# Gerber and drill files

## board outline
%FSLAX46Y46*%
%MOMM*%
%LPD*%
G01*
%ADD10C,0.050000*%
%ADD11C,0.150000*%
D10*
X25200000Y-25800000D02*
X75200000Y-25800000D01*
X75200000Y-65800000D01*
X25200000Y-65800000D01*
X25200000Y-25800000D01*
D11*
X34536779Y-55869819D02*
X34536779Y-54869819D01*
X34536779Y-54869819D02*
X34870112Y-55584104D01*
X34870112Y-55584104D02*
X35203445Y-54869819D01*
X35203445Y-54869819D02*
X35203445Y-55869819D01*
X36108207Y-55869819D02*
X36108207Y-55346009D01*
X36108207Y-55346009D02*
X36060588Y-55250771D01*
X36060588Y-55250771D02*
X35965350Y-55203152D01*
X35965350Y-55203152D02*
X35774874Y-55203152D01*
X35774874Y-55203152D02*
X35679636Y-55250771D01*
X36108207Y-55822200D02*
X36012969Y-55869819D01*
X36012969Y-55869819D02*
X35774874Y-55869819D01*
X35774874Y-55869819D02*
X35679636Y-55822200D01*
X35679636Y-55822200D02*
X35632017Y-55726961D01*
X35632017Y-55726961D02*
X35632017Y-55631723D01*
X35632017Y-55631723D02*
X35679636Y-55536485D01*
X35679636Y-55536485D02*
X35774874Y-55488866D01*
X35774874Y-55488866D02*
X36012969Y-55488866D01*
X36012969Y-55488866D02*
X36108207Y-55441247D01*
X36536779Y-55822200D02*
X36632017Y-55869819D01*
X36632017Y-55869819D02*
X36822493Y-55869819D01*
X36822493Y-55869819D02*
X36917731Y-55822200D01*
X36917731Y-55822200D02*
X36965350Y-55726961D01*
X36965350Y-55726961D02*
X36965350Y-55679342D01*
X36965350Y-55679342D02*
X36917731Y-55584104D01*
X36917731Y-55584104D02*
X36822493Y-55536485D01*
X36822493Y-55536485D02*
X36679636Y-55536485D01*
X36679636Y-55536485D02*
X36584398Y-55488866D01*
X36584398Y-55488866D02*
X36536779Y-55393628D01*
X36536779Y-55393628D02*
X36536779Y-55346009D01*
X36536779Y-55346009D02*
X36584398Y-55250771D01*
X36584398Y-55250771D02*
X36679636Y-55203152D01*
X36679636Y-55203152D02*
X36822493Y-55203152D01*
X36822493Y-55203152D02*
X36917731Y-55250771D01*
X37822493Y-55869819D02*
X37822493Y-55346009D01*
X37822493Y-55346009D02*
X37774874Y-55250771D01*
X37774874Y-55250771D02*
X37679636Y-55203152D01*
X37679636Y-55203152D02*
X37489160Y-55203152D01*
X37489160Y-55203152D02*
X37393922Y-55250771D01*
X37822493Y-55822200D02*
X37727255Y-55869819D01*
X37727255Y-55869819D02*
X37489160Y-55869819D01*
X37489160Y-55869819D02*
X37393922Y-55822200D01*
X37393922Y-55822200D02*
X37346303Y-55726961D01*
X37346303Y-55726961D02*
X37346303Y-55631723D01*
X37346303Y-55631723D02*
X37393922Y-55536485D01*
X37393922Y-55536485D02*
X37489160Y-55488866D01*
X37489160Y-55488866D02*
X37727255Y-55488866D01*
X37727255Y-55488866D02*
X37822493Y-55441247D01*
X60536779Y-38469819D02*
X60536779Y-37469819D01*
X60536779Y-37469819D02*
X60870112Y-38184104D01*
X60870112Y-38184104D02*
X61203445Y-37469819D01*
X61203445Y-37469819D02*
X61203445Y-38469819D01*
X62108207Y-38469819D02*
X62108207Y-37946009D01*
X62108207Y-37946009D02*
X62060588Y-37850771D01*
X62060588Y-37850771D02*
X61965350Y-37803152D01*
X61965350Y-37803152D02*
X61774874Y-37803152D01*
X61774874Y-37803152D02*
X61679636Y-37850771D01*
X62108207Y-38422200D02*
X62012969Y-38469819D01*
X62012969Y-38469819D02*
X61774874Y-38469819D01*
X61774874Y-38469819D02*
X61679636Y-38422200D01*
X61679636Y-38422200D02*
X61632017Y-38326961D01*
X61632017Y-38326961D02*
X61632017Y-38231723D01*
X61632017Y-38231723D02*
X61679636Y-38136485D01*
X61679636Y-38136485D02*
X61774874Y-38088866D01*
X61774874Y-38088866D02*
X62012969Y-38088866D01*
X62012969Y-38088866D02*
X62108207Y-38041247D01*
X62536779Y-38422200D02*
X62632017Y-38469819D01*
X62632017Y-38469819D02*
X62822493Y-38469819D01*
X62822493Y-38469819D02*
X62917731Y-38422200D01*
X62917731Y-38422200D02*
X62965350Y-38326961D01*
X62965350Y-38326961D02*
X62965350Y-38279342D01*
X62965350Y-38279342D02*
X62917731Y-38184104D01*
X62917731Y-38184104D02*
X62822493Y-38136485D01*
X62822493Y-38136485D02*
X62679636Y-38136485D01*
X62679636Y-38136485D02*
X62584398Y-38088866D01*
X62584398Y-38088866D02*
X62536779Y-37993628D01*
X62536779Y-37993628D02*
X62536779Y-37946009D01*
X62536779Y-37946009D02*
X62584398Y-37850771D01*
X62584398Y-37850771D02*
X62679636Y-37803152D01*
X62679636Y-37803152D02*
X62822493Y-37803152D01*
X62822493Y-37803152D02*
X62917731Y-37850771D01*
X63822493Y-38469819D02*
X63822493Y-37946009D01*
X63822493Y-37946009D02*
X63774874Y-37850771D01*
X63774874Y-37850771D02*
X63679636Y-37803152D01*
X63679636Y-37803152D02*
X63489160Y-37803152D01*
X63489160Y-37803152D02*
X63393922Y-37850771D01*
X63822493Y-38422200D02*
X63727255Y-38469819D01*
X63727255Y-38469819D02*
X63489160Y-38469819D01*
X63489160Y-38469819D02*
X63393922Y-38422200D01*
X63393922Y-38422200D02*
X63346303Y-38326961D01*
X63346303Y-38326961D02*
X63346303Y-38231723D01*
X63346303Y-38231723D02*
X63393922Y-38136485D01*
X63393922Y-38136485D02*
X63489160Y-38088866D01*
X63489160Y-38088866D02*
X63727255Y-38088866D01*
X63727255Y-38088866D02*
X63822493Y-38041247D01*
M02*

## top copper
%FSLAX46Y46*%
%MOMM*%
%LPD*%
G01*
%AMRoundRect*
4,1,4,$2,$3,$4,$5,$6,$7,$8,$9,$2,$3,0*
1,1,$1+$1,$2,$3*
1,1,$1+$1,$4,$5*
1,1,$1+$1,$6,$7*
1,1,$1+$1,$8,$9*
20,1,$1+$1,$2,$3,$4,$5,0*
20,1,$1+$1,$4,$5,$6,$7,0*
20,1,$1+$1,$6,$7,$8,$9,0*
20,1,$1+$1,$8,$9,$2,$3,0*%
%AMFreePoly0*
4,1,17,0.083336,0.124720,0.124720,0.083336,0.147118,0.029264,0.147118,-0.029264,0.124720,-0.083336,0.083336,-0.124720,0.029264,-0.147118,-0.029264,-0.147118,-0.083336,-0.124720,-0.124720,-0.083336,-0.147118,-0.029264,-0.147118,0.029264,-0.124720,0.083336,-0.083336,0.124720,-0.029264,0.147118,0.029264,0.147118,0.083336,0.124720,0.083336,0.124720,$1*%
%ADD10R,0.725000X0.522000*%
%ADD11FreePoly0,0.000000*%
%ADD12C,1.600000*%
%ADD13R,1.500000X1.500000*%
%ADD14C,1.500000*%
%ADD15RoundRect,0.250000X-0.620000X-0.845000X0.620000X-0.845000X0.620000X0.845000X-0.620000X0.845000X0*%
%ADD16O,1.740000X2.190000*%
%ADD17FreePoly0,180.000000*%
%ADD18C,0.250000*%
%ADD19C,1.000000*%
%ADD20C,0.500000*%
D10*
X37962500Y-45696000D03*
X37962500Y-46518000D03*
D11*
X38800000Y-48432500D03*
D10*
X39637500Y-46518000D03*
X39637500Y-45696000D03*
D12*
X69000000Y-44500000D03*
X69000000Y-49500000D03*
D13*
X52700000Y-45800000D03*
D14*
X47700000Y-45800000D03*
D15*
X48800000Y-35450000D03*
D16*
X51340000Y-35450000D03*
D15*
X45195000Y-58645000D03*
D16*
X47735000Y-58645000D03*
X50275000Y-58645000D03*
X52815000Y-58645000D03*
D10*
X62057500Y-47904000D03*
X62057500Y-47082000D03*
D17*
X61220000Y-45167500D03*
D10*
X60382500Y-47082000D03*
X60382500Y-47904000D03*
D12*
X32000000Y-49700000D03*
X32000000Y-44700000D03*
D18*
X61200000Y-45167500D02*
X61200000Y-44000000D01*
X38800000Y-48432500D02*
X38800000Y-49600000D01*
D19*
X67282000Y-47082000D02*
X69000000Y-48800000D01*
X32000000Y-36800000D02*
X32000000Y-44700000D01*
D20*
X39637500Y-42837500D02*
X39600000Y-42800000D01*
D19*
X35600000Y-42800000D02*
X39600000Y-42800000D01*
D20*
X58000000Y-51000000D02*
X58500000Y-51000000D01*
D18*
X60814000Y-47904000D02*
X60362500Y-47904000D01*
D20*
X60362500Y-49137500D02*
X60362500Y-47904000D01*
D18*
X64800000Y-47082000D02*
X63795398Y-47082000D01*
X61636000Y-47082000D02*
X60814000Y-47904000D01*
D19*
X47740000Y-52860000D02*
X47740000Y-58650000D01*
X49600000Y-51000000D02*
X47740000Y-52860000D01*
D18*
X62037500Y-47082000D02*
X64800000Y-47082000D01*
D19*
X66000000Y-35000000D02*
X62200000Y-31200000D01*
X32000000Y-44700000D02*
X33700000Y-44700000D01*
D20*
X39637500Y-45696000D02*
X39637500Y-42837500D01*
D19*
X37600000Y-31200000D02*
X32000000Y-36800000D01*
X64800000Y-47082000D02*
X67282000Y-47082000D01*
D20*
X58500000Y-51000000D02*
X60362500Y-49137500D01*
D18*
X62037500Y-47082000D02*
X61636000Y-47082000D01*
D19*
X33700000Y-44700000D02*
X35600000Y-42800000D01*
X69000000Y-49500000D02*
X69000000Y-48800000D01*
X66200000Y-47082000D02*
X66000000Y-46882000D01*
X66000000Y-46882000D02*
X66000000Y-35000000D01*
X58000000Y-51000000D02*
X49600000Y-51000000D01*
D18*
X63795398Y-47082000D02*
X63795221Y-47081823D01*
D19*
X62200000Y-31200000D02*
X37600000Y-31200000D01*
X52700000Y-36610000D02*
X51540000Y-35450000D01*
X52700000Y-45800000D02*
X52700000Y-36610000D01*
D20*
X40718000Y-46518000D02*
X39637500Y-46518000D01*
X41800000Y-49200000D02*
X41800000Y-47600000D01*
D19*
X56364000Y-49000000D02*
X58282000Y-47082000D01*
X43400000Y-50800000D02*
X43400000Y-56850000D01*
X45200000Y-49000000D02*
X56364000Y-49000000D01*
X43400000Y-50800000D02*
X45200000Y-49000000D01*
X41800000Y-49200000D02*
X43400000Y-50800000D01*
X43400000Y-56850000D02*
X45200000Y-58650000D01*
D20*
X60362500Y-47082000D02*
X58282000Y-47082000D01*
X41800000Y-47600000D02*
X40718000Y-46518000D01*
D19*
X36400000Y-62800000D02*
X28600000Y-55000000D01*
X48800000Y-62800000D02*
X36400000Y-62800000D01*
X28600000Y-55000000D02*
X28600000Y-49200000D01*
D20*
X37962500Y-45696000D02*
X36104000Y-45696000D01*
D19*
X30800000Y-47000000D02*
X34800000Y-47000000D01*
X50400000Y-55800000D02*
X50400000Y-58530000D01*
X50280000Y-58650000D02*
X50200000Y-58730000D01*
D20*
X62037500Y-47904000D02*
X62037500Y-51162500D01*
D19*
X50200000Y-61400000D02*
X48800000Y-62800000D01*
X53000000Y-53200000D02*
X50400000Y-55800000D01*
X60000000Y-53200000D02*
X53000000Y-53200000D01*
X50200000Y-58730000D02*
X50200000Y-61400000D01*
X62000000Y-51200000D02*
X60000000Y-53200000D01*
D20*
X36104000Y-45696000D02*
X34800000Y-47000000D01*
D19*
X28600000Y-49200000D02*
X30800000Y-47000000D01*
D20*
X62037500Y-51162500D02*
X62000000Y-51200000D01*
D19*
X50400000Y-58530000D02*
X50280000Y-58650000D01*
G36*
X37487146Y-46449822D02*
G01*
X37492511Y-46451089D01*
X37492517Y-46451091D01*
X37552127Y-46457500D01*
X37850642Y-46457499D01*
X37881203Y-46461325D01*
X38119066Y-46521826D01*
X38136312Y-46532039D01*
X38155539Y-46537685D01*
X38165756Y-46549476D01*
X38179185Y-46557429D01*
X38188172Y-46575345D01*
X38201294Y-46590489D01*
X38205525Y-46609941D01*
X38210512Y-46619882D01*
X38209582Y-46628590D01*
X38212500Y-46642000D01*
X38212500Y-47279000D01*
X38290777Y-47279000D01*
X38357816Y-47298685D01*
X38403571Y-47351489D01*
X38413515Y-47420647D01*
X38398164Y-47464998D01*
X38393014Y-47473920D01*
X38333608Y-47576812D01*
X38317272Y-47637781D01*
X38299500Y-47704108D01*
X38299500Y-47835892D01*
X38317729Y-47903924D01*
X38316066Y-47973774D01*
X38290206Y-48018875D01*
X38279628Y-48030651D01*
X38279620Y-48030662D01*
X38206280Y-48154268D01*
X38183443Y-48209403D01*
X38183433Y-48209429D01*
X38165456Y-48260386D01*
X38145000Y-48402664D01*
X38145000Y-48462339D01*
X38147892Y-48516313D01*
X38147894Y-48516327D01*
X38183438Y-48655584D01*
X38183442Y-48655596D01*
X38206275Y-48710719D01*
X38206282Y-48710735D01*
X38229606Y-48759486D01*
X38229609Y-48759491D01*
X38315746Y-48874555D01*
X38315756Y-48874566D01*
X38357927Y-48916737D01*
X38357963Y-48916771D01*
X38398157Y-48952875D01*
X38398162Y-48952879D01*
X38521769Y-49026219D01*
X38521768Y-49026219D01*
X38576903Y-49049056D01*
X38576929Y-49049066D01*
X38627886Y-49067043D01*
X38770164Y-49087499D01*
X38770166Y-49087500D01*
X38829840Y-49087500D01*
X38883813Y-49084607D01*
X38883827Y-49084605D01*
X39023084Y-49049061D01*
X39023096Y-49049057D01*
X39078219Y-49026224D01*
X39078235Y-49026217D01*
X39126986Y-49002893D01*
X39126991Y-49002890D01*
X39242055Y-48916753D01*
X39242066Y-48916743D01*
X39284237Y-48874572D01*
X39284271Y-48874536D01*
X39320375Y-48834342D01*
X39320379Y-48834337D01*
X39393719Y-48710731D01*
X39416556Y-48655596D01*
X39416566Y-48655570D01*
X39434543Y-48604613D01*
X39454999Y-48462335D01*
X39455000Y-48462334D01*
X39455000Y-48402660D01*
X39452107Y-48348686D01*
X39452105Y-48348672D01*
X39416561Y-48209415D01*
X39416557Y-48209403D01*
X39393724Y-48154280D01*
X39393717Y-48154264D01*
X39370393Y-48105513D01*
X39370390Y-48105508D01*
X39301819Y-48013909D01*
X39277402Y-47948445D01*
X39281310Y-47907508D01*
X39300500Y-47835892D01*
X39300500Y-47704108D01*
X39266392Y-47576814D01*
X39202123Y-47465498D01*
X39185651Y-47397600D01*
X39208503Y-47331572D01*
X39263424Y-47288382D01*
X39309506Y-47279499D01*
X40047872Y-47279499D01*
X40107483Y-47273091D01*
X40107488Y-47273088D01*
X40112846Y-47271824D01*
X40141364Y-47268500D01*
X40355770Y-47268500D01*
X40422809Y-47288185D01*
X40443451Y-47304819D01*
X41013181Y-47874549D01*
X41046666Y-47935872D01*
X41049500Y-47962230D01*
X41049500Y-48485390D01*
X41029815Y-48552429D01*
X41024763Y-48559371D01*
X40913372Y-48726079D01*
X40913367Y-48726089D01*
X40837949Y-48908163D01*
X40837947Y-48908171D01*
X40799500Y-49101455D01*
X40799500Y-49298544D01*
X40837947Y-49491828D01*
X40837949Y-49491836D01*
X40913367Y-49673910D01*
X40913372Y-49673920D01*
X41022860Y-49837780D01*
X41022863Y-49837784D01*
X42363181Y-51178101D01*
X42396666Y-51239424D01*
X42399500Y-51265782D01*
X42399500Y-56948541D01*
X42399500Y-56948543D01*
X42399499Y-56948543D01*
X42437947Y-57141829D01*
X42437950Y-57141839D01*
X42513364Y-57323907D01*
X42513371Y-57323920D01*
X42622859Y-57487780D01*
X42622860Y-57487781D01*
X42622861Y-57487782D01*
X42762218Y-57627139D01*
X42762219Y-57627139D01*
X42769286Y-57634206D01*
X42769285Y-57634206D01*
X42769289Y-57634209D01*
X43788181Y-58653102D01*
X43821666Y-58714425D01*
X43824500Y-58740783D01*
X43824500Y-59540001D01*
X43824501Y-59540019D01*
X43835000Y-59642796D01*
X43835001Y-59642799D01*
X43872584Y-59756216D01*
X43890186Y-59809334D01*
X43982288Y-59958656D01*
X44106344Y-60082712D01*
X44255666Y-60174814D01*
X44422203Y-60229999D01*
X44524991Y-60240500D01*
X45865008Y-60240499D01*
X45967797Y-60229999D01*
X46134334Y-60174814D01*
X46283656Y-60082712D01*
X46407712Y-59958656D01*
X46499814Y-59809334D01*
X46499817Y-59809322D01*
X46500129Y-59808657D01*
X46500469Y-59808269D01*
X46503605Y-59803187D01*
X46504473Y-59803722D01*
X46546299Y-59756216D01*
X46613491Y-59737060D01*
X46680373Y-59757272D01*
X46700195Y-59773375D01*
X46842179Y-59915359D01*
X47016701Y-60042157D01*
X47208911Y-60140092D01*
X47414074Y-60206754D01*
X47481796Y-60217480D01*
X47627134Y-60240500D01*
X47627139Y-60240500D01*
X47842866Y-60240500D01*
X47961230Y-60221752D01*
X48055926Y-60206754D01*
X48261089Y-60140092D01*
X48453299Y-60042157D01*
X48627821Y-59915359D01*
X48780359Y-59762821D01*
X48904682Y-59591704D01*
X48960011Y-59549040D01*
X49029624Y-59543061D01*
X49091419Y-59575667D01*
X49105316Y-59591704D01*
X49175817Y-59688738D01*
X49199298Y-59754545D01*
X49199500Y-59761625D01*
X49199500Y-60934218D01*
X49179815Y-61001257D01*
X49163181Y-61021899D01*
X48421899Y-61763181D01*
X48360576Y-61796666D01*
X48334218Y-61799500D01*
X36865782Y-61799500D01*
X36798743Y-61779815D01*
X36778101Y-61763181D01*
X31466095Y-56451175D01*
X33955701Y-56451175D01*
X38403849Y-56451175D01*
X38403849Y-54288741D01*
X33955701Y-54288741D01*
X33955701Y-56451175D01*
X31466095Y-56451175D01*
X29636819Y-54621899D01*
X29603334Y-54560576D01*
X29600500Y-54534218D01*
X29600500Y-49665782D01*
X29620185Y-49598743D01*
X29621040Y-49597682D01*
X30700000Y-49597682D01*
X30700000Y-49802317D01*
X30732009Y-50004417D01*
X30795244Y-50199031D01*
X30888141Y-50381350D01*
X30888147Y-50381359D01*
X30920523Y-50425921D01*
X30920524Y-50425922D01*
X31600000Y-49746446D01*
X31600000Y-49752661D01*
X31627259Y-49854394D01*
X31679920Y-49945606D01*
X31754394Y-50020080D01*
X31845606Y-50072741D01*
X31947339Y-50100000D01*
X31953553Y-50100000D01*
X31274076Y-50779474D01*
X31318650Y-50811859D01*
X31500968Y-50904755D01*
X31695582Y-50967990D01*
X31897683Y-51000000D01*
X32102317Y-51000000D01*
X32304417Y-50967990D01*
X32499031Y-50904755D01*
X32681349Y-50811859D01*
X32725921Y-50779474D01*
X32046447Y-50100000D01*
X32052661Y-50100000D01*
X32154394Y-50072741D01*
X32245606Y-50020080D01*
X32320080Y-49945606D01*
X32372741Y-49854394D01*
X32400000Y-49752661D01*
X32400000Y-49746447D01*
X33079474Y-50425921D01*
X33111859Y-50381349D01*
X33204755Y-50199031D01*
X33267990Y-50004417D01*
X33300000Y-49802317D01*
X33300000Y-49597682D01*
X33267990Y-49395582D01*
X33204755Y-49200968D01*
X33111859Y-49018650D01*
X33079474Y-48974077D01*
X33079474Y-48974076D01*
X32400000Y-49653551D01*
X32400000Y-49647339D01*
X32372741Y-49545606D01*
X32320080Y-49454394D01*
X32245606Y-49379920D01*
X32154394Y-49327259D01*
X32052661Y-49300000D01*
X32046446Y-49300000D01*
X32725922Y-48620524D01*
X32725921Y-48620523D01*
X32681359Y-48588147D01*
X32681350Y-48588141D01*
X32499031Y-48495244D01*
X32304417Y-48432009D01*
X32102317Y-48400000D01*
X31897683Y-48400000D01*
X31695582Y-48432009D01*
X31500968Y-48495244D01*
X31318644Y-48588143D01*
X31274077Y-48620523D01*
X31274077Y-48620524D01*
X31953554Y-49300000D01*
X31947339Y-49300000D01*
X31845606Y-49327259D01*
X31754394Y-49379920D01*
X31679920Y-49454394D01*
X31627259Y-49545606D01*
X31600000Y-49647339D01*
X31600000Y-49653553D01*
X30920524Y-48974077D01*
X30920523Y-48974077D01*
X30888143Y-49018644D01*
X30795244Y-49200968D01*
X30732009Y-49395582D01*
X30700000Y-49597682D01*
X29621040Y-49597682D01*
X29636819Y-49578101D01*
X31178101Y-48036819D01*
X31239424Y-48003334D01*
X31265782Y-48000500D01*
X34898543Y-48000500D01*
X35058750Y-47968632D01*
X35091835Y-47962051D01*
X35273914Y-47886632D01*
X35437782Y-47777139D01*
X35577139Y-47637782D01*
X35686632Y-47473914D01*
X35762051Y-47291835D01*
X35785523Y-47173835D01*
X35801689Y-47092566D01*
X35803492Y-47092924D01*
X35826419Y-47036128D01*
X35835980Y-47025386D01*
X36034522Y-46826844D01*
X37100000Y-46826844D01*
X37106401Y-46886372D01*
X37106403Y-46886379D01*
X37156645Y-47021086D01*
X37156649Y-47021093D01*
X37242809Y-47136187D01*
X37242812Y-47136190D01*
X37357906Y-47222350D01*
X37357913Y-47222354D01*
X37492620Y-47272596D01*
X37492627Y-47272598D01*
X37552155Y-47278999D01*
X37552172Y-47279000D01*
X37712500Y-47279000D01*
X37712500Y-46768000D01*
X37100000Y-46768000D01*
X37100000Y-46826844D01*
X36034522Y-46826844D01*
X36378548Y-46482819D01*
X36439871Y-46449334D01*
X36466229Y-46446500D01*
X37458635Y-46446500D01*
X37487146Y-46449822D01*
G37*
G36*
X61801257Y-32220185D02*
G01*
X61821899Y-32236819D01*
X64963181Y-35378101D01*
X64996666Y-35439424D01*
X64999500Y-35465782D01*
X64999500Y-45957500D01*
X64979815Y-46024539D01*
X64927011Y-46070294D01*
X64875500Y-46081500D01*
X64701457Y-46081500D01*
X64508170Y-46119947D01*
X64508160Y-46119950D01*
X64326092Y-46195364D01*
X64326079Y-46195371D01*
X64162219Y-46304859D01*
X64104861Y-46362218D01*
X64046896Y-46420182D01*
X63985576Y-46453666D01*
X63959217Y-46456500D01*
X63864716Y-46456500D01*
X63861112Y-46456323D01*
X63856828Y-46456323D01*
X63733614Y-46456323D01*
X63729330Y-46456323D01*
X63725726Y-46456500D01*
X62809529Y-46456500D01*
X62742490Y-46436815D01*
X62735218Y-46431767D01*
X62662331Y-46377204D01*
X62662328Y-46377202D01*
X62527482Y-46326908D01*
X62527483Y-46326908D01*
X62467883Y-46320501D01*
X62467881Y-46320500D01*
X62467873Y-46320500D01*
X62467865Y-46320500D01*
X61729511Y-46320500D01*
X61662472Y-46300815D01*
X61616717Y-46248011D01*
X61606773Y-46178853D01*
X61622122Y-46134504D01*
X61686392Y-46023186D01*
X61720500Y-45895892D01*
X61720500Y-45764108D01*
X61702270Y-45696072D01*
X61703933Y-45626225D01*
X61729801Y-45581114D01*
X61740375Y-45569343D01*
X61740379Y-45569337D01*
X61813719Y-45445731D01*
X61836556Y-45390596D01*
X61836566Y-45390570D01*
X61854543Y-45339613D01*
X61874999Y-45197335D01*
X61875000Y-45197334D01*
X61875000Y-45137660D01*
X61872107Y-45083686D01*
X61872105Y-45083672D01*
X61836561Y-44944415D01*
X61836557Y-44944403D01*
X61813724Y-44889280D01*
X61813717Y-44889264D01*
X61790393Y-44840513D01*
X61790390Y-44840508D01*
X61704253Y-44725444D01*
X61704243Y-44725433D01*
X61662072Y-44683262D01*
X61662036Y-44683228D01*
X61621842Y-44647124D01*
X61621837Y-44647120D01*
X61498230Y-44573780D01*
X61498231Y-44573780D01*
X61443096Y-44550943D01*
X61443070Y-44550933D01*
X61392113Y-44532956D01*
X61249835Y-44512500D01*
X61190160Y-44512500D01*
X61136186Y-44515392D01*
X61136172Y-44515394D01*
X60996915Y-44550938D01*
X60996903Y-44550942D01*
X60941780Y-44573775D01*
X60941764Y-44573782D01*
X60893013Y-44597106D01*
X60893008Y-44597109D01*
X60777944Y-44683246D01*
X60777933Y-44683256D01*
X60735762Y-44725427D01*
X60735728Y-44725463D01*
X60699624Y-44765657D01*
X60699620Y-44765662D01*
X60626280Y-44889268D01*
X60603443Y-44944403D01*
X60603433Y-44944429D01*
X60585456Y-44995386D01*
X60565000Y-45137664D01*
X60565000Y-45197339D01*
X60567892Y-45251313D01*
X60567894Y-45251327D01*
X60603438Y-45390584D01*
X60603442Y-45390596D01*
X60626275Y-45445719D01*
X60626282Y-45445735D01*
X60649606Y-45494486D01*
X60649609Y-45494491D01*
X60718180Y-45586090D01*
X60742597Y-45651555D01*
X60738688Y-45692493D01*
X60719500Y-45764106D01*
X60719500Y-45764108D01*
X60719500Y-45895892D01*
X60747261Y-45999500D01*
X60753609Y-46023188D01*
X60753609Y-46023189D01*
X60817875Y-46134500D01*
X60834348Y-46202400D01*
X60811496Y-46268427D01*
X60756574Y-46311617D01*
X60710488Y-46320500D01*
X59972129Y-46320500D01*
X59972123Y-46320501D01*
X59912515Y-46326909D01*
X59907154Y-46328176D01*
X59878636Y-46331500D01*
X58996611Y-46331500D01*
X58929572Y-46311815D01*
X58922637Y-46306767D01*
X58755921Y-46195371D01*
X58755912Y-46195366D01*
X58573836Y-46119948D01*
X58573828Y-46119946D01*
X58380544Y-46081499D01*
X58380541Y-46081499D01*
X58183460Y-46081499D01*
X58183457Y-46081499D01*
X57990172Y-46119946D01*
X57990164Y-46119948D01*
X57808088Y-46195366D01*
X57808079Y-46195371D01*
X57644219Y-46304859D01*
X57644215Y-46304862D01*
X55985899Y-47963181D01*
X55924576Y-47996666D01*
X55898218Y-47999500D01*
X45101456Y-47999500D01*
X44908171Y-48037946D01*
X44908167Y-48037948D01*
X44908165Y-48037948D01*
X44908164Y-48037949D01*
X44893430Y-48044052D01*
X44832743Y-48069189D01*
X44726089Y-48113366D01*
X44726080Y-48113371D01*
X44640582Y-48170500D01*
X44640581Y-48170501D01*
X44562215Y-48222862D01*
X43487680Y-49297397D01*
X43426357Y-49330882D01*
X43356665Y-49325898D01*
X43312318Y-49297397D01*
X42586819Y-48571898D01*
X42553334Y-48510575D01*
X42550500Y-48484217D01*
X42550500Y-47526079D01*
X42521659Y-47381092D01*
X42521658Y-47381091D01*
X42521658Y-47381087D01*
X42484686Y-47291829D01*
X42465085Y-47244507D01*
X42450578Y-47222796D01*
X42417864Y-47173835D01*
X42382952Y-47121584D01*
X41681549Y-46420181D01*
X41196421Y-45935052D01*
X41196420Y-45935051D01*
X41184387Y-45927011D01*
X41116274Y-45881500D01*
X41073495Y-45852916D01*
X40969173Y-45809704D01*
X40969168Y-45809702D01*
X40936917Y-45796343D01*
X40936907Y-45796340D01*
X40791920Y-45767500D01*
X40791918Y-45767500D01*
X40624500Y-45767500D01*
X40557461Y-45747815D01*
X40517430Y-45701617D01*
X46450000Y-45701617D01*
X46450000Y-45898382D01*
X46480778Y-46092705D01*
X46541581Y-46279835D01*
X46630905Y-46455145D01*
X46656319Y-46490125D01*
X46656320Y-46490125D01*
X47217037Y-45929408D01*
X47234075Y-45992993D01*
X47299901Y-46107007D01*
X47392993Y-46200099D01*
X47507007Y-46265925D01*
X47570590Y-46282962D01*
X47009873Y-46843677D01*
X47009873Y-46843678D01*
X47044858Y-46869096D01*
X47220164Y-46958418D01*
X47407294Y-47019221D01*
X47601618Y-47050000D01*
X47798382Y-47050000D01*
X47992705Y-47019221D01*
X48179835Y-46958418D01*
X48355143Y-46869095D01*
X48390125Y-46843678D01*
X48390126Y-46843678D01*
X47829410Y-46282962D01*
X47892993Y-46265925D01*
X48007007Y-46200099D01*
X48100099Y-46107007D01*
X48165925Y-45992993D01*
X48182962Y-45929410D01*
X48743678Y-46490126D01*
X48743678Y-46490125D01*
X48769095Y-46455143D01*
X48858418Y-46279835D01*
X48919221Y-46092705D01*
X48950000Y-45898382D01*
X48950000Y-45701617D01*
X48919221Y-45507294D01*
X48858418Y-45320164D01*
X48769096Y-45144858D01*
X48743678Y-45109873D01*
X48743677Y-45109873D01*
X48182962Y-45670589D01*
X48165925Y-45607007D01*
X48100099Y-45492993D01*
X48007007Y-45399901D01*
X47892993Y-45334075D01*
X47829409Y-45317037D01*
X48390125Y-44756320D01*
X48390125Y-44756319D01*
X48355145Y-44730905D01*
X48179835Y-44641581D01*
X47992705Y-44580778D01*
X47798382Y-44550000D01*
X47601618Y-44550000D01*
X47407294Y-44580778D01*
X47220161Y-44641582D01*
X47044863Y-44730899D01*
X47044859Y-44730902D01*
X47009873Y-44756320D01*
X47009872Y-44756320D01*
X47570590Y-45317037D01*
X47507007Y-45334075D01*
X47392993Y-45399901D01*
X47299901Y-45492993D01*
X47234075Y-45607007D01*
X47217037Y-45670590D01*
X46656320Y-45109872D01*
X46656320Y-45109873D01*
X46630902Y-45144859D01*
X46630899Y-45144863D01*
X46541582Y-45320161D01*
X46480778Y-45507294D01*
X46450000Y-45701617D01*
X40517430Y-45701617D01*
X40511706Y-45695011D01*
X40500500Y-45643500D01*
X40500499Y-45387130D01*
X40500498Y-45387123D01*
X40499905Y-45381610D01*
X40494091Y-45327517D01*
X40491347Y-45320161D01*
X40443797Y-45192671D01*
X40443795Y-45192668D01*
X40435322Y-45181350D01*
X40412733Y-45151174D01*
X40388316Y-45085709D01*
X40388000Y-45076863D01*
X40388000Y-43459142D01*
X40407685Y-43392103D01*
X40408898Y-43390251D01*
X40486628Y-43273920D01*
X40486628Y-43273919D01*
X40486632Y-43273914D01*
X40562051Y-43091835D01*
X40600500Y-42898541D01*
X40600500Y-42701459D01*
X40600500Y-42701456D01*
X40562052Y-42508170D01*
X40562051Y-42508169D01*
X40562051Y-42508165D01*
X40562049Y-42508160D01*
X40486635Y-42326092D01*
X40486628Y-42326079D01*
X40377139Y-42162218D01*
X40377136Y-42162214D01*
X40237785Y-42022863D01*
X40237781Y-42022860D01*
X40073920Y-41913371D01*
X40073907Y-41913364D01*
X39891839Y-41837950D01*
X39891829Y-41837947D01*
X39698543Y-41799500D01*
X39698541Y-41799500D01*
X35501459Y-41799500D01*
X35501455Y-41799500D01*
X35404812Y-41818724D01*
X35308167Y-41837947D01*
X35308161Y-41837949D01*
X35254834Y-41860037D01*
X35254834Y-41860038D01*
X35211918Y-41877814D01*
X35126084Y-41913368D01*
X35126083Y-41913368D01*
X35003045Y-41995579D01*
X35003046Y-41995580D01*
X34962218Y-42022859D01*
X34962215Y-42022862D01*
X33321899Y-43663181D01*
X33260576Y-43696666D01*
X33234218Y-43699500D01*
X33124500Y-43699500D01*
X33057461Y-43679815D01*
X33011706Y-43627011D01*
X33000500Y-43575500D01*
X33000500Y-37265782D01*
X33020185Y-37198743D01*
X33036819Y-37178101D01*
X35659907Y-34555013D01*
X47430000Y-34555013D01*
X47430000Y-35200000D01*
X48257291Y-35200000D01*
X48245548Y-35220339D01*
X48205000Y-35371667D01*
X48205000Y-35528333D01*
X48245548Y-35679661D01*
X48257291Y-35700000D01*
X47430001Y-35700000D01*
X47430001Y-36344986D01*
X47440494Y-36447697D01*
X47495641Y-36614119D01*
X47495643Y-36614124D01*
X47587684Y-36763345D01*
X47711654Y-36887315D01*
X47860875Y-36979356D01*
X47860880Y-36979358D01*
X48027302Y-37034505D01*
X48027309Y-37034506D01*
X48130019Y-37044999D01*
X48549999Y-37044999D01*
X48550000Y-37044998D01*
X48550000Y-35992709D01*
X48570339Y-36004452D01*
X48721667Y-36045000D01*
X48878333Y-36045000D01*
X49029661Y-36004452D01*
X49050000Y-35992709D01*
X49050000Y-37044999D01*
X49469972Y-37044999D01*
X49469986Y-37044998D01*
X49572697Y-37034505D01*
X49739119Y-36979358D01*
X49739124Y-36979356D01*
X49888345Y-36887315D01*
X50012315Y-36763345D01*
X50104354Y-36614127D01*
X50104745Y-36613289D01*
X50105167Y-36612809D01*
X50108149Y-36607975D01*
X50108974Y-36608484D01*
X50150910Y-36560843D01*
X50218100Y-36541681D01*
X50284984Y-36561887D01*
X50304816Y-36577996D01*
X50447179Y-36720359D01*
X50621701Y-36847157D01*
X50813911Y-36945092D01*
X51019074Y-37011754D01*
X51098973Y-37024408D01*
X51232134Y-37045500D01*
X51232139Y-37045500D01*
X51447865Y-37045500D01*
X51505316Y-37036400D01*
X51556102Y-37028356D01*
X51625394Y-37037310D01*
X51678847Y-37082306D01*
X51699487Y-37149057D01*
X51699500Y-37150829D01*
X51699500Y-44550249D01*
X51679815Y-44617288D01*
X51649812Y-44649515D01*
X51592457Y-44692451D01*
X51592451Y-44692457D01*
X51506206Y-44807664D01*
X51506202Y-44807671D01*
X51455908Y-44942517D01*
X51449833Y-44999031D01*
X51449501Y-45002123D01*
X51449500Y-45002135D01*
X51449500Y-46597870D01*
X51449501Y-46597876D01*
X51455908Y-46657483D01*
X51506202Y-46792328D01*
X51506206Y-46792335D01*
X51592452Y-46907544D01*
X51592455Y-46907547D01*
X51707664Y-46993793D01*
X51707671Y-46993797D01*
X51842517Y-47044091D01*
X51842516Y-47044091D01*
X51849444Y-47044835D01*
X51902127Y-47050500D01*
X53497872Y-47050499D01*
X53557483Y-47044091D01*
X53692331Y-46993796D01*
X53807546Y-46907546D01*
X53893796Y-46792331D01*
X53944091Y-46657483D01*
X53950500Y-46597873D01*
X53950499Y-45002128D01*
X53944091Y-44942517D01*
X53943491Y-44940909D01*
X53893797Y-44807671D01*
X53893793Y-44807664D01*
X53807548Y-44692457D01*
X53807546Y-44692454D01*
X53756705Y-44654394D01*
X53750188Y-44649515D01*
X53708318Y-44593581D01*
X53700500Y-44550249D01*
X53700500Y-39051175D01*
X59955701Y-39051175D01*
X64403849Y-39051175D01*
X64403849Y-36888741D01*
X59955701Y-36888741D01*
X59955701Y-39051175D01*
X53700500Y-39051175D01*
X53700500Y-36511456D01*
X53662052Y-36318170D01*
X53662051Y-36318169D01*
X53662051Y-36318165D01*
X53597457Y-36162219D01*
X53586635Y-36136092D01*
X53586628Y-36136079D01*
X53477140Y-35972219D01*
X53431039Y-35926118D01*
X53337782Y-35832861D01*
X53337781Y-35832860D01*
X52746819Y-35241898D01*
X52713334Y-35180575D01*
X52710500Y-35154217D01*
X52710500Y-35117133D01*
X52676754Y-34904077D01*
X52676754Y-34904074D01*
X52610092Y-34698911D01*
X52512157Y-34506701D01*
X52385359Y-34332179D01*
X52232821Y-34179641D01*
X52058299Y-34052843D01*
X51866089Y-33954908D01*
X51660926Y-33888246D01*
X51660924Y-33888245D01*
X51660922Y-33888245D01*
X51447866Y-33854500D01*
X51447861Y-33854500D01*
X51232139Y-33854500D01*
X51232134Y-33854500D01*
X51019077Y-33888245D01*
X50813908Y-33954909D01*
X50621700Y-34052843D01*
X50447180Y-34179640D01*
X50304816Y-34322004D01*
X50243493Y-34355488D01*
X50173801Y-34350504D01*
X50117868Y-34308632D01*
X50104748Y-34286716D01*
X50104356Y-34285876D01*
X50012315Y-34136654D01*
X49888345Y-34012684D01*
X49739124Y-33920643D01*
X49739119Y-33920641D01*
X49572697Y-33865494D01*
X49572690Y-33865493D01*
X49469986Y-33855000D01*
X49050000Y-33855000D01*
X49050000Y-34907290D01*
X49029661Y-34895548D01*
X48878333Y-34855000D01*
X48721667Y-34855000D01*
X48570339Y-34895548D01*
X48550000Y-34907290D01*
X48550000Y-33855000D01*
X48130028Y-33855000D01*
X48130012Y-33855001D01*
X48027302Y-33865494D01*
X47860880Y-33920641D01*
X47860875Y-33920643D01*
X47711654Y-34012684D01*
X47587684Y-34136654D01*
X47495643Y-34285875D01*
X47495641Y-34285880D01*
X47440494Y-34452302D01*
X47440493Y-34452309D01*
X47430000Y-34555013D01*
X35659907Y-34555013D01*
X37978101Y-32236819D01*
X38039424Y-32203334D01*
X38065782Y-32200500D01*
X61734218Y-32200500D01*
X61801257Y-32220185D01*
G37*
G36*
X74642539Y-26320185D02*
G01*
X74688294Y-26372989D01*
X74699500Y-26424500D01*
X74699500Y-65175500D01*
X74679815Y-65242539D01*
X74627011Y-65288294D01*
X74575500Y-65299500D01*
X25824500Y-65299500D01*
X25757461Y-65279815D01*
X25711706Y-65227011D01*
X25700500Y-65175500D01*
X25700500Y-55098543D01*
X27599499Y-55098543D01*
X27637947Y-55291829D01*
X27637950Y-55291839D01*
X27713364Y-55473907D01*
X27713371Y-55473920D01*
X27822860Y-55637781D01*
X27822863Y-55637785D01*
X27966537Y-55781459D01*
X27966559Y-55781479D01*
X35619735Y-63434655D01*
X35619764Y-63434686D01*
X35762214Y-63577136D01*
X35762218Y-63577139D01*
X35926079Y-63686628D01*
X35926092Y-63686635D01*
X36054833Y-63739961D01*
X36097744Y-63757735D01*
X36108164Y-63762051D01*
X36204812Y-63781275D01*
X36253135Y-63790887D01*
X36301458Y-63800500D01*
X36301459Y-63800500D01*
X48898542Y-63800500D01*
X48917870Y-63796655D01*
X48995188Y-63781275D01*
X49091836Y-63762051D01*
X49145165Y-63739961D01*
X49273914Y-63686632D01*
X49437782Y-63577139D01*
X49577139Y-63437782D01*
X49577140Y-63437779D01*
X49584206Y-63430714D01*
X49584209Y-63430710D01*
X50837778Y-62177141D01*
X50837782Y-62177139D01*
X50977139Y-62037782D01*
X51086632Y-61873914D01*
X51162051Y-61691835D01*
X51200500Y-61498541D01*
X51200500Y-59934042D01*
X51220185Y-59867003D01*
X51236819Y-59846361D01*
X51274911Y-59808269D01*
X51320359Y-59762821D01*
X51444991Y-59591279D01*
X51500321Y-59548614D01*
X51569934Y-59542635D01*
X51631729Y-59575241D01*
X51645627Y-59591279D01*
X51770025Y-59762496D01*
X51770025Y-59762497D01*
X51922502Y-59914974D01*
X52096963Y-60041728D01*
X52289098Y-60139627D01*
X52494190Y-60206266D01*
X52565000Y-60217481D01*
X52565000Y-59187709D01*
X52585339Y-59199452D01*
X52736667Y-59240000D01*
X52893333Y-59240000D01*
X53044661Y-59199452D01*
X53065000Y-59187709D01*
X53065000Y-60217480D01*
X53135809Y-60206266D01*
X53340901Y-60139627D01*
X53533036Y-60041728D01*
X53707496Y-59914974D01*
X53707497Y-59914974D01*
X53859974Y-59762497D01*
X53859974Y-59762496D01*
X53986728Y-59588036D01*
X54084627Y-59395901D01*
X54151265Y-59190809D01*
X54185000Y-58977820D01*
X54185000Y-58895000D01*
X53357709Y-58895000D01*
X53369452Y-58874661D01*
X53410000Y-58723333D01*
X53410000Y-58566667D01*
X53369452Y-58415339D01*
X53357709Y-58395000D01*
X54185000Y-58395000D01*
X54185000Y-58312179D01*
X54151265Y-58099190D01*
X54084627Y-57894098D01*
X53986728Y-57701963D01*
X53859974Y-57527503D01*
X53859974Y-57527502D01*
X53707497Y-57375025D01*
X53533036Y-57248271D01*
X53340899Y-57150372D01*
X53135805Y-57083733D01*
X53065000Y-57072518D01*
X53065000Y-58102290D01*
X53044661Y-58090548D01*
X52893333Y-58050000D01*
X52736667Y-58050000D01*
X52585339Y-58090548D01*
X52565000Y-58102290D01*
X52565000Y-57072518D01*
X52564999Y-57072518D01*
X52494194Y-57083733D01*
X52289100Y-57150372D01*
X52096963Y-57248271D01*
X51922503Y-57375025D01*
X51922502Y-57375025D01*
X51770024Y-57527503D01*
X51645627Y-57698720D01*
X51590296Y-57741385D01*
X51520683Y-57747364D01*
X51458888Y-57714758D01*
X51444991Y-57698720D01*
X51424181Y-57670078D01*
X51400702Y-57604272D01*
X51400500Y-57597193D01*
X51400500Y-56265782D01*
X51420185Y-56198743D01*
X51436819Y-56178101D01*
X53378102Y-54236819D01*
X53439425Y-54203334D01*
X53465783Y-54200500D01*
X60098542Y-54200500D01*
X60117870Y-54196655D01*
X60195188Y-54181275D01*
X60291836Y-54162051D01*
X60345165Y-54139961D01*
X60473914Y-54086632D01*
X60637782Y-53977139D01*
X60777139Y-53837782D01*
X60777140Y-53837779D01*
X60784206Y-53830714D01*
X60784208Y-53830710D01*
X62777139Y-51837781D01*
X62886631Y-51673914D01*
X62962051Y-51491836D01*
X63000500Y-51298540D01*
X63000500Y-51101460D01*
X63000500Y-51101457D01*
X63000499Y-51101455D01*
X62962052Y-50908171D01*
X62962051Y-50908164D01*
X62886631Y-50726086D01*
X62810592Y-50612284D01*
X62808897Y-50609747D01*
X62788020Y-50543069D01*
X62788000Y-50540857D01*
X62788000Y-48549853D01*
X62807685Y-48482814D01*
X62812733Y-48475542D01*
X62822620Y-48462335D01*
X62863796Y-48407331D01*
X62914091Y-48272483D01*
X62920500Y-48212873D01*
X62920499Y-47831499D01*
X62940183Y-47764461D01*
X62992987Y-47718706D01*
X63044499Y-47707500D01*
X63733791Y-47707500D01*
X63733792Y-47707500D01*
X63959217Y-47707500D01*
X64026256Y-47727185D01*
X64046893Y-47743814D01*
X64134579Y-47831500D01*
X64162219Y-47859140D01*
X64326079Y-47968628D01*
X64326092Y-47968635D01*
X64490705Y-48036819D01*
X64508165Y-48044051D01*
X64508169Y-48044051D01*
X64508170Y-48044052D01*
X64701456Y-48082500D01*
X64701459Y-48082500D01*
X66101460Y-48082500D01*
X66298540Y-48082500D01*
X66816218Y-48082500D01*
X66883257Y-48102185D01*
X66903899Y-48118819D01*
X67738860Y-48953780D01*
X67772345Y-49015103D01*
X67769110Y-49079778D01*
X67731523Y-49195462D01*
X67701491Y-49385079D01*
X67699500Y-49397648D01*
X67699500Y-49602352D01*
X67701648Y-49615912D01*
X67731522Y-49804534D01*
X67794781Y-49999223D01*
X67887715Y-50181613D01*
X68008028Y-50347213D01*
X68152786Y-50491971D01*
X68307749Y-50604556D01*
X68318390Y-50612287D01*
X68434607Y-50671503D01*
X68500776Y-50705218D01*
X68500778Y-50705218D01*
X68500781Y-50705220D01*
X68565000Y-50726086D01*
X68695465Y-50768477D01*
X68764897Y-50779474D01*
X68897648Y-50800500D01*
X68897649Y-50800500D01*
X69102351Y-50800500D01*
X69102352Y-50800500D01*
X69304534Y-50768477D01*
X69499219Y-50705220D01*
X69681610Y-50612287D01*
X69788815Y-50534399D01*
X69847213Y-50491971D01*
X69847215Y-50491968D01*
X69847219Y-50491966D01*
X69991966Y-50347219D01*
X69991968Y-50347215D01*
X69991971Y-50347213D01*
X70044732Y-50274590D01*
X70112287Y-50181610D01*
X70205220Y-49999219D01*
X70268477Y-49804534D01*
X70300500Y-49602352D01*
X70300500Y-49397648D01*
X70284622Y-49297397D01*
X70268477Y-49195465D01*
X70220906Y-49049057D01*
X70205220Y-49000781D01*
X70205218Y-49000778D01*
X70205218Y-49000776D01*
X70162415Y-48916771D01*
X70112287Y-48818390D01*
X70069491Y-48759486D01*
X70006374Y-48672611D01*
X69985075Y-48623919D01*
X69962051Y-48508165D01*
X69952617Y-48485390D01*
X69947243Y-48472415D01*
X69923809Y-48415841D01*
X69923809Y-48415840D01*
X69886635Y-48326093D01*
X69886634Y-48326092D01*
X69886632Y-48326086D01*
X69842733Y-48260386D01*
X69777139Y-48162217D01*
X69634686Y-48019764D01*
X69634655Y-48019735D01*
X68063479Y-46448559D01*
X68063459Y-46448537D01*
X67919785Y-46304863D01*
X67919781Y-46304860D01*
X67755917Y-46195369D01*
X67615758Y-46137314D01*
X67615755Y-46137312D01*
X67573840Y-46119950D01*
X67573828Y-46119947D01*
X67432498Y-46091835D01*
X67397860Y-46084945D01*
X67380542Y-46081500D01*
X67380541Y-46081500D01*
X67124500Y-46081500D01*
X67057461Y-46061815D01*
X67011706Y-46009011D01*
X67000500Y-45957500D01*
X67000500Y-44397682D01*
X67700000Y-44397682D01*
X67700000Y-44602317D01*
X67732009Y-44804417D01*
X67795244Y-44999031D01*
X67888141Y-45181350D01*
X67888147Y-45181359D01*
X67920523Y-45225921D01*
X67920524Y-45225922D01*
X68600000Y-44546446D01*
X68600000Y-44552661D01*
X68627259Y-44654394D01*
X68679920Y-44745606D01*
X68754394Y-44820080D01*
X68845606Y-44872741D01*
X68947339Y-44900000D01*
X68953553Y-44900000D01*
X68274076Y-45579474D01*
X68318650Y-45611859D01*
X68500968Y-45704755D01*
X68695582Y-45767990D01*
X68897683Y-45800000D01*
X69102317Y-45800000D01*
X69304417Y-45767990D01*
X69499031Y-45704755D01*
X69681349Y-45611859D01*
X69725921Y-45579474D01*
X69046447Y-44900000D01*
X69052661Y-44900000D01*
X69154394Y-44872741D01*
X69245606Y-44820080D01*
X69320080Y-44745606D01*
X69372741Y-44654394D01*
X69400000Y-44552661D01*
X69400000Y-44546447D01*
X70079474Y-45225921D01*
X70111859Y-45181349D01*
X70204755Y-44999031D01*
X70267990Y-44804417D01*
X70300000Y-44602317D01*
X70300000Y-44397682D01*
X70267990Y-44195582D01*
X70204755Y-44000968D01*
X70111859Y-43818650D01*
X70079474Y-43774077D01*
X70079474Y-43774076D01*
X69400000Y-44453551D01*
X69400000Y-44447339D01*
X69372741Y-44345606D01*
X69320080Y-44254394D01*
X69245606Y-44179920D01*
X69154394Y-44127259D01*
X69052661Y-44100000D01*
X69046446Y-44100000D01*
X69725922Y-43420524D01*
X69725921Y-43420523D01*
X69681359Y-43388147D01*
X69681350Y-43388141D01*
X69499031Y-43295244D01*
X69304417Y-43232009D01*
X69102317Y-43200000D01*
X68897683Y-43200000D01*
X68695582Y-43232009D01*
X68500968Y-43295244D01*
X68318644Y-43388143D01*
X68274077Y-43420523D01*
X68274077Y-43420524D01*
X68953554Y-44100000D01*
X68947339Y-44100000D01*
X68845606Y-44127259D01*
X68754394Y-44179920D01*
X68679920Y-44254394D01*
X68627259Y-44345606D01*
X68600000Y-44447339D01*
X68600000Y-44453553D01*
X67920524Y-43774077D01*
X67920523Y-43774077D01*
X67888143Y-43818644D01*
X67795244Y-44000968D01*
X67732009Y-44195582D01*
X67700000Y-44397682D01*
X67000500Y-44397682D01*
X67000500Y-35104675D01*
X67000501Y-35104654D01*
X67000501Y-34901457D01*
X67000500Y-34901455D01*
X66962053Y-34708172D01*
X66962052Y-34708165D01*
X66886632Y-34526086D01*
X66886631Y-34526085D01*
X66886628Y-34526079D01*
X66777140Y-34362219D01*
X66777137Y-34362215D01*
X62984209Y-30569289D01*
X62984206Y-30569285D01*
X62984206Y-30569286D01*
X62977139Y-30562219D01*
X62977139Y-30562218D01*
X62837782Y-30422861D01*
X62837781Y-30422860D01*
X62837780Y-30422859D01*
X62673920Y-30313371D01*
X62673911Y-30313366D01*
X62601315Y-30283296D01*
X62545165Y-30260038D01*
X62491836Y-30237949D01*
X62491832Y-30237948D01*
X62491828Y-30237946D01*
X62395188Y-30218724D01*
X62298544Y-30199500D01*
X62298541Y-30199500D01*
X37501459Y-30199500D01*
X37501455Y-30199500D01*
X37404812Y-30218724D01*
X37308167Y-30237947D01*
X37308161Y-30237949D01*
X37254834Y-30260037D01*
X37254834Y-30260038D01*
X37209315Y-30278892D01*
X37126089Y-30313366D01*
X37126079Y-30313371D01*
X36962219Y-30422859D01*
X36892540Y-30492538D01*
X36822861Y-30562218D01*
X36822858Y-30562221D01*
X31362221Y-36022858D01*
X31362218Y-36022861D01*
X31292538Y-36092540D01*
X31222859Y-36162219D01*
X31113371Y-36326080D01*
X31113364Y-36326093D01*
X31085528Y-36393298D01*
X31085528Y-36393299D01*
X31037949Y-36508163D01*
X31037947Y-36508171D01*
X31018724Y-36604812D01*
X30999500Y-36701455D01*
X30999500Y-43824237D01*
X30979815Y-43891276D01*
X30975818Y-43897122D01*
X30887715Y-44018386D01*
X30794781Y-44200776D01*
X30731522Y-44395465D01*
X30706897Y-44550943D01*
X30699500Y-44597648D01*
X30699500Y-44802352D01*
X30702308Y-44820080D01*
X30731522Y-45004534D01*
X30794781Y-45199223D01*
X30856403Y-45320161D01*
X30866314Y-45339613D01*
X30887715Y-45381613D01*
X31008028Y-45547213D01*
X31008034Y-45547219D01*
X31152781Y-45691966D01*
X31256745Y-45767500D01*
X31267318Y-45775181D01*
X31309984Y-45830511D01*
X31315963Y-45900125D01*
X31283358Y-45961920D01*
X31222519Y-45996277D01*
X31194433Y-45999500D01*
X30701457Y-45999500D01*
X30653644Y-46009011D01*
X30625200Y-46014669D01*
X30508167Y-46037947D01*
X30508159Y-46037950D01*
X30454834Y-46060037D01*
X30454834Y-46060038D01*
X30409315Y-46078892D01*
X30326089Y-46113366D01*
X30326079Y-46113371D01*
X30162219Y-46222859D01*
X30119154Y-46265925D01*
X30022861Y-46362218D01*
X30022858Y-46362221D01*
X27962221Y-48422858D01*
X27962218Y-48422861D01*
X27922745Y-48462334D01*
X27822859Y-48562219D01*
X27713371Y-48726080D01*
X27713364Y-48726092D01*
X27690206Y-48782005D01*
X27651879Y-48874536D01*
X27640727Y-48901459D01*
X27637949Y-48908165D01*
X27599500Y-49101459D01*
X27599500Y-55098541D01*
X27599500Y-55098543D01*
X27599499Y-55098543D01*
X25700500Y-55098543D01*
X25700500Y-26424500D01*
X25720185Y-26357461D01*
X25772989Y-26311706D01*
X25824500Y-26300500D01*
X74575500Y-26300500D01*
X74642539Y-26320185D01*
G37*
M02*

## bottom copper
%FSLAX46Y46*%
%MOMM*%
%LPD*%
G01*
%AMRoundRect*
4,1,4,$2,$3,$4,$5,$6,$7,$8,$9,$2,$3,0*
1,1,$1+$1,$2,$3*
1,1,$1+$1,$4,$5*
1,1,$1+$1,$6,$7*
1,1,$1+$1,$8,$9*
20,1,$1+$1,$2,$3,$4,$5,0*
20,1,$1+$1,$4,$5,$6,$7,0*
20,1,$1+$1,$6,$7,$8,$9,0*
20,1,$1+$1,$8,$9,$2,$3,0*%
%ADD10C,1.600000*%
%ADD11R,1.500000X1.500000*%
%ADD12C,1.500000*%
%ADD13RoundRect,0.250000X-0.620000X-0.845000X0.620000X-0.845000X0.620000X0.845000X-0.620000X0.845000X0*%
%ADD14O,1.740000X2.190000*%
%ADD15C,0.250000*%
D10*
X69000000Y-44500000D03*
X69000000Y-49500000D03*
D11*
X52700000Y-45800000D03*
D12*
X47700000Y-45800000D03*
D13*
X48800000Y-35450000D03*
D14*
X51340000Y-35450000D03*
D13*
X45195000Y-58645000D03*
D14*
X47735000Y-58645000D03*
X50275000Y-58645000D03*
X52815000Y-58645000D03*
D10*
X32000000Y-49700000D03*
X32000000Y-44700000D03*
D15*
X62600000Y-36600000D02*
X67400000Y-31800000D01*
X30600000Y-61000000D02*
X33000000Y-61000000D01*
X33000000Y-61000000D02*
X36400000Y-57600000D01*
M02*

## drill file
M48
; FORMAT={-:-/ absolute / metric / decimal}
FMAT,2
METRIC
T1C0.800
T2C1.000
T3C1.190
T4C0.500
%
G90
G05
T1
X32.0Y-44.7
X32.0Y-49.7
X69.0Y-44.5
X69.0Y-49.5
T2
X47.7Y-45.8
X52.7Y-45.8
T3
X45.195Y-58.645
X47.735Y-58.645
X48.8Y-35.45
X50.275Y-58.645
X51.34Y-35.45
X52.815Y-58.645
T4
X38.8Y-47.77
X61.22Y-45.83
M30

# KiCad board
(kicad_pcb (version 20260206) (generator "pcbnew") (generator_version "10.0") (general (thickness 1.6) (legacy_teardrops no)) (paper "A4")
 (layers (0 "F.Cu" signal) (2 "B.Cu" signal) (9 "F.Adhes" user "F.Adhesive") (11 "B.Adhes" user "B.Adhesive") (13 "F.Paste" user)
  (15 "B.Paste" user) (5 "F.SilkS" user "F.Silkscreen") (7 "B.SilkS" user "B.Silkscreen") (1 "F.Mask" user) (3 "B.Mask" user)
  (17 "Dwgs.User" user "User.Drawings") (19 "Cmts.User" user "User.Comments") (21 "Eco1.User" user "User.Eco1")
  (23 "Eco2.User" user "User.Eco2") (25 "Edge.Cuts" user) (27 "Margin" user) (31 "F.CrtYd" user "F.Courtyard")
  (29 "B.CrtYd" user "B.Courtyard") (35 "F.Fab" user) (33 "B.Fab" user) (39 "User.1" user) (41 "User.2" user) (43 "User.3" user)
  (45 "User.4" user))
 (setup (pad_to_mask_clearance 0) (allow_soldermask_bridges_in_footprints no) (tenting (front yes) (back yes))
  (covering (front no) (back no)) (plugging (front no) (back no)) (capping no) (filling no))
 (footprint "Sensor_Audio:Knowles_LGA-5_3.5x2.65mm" (layer "F.Cu") (at 38.8 47)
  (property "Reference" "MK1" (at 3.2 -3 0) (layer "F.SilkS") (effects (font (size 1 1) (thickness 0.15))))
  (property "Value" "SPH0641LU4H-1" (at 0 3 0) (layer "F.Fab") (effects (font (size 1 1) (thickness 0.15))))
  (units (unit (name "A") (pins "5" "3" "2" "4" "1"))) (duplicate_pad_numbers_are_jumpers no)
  (pad "" np_thru_hole circle (at 0 0.77) (size 0.5 0.5) (drill 0.5) (layers "*.Cu" "*.Mask"))
  (pad "1" smd rect (at -0.8375 -1.304) (size 0.725 0.522) (layers "F.Cu" "F.Mask" "F.Paste") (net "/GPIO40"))
  (pad "2" smd rect (at -0.8375 -0.482) (size 0.725 0.522) (layers "F.Cu" "F.Mask" "F.Paste") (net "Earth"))
  (pad "3" smd custom (at 0 1.4325) (size 0.3 0.3) (layers "F.Cu" "F.Mask") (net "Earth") (zone_connect 0)
   (options (clearance outline) (anchor circle)) (primitives))
  (pad "4" smd rect (at 0.8375 -0.482) (size 0.725 0.522) (layers "F.Cu" "F.Mask" "F.Paste") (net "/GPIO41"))
  (pad "5" smd rect (at 0.8375 -1.304) (size 0.725 0.522) (layers "F.Cu" "F.Mask" "F.Paste") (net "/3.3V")))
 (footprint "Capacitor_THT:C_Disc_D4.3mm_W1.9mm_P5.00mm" (layer "F.Cu") (at 69 44.5 -90)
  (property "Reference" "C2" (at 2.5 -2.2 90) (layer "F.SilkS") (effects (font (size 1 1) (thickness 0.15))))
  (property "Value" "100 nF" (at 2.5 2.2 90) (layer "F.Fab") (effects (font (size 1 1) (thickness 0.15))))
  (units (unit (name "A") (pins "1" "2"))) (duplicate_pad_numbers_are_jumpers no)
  (pad "1" thru_hole circle (at 0 0 270) (size 1.6 1.6) (drill 0.8) (layers "*.Cu" "*.Mask") (remove_unused_layers no) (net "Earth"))
  (pad "2" thru_hole circle (at 5 0 270) (size 1.6 1.6) (drill 0.8) (layers "*.Cu" "*.Mask") (remove_unused_layers no) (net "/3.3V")))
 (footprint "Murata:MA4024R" (layer "F.Cu") (at 50.2 45.8 180)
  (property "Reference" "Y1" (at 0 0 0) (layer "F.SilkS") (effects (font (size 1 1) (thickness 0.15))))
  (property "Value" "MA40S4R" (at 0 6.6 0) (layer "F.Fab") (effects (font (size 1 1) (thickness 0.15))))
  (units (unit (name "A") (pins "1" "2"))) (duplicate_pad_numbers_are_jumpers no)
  (pad "1" thru_hole rect (at -2.5 0 180) (size 1.5 1.5) (drill 1) (layers "*.Cu" "*.Mask") (remove_unused_layers no)
   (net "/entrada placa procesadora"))
  (pad "2" thru_hole circle (at 2.5 0 180) (size 1.5 1.5) (drill 1) (layers "*.Cu" "*.Mask") (remove_unused_layers no) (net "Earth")))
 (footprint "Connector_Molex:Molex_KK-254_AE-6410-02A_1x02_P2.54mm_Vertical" (layer "F.Cu") (at 48.8 35.45)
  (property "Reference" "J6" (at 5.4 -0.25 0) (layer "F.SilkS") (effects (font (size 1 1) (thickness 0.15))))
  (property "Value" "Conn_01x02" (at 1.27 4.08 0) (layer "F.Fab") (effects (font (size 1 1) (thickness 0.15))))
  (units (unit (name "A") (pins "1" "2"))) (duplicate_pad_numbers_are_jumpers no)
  (pad "1" thru_hole roundrect (at 0 0) (size 1.74 2.19) (drill 1.19) (layers "*.Cu" "*.Mask") (remove_unused_layers no)
   (roundrect_rratio 0.143678) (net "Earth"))
  (pad "2" thru_hole oval (at 2.54 0) (size 1.74 2.19) (drill 1.19) (layers "*.Cu" "*.Mask") (remove_unused_layers no)
   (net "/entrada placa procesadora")))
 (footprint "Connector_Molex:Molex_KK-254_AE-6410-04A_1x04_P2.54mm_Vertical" (layer "F.Cu") (at 45.195 58.645)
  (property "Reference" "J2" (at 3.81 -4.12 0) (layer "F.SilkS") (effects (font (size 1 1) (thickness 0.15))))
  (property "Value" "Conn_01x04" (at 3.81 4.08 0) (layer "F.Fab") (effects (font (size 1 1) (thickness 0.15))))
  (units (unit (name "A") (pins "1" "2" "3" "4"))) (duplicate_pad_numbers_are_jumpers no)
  (pad "1" thru_hole roundrect (at 0 0) (size 1.74 2.19) (drill 1.19) (layers "*.Cu" "*.Mask") (remove_unused_layers no)
   (roundrect_rratio 0.143678) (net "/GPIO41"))
  (pad "2" thru_hole oval (at 2.54 0) (size 1.74 2.19) (drill 1.19) (layers "*.Cu" "*.Mask") (remove_unused_layers no) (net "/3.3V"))
  (pad "3" thru_hole oval (at 5.08 0) (size 1.74 2.19) (drill 1.19) (layers "*.Cu" "*.Mask") (remove_unused_layers no) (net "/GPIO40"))
  (pad "4" thru_hole oval (at 7.62 0) (size 1.74 2.19) (drill 1.19) (layers "*.Cu" "*.Mask") (remove_unused_layers no) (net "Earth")))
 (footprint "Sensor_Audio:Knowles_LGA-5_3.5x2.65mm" (layer "F.Cu") (at 61.22 46.6 180)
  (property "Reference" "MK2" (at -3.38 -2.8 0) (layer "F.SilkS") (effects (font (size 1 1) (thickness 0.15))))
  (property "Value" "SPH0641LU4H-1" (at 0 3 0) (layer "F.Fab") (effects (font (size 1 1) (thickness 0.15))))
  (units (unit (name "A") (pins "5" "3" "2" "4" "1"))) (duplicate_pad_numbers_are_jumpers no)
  (pad "" np_thru_hole circle (at 0 0.77 180) (size 0.5 0.5) (drill 0.5) (layers "*.Cu" "*.Mask"))
  (pad "1" smd rect (at -0.8375 -1.304 180) (size 0.725 0.522) (layers "F.Cu" "F.Mask" "F.Paste") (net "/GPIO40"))
  (pad "2" smd rect (at -0.8375 -0.482 180) (size 0.725 0.522) (layers "F.Cu" "F.Mask" "F.Paste") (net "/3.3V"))
  (pad "3" smd custom (at 0 1.4325 180) (size 0.3 0.3) (layers "F.Cu" "F.Mask") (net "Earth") (zone_connect 0)
   (options (clearance outline) (anchor circle)) (primitives))
  (pad "4" smd rect (at 0.8375 -0.482 180) (size 0.725 0.522) (layers "F.Cu" "F.Mask" "F.Paste") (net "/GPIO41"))
  (pad "5" smd rect (at 0.8375 -1.304 180) (size 0.725 0.522) (layers "F.Cu" "F.Mask" "F.Paste") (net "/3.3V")))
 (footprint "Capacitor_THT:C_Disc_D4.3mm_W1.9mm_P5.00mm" (layer "F.Cu") (at 32 49.7 90)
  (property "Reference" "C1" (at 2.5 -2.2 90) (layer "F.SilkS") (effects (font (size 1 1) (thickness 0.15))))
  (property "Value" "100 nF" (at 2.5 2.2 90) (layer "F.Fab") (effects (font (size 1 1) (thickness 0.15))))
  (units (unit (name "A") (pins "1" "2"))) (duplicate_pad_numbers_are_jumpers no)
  (pad "1" thru_hole circle (at 0 0 90) (size 1.6 1.6) (drill 0.8) (layers "*.Cu" "*.Mask") (remove_unused_layers no) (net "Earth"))
  (pad "2" thru_hole circle (at 5 0 90) (size 1.6 1.6) (drill 0.8) (layers "*.Cu" "*.Mask") (remove_unused_layers no) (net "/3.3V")))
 (gr_rect (start 25.2 25.8) (end 75.2 65.8) (stroke (width 0.05) (type solid)) (fill no) (layer "Edge.Cuts"))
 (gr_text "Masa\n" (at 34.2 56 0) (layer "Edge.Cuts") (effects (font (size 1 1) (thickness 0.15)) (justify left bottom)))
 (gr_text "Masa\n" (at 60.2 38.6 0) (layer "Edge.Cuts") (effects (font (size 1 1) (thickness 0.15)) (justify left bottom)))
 (segment (start 62.6 36.6) (end 67.4 31.8) (width 0.25) (layer "B.Cu") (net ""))
 (segment (start 30.6 61) (end 33 61) (width 0.25) (layer "B.Cu") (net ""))
 (segment (start 33 61) (end 36.4 57.6) (width 0.25) (layer "B.Cu") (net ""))
 (segment (start 61.2 45.1675) (end 61.2 44) (width 0.25) (layer "F.Cu") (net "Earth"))
 (segment (start 38.8 48.4325) (end 38.8 49.6) (width 0.25) (layer "F.Cu") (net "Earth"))
 (segment (start 67.282 47.082) (end 69 48.8) (width 1) (layer "F.Cu") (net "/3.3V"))
 (segment (start 32 36.8) (end 32 44.7) (width 1) (layer "F.Cu") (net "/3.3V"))
 (segment (start 39.6375 42.8375) (end 39.6 42.8) (width 0.5) (layer "F.Cu") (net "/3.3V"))
 (segment (start 35.6 42.8) (end 39.6 42.8) (width 1) (layer "F.Cu") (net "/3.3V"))
 (segment (start 58 51) (end 58.5 51) (width 0.5) (layer "F.Cu") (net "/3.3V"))
 (segment (start 60.814 47.904) (end 60.3625 47.904) (width 0.25) (layer "F.Cu") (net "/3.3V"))
 (segment (start 60.3625 49.1375) (end 60.3625 47.904) (width 0.5) (layer "F.Cu") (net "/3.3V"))
 (segment (start 64.8 47.082) (end 63.795398 47.082) (width 0.25) (layer "F.Cu") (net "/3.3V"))
 (segment (start 61.636 47.082) (end 60.814 47.904) (width 0.25) (layer "F.Cu") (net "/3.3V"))
 (segment (start 47.74 52.86) (end 47.74 58.65) (width 1) (layer "F.Cu") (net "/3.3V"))
 (segment (start 49.6 51) (end 47.74 52.86) (width 1) (layer "F.Cu") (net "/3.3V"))
 (segment (start 62.0375 47.082) (end 64.8 47.082) (width 0.25) (layer "F.Cu") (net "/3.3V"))
 (segment (start 66 35) (end 62.2 31.2) (width 1) (layer "F.Cu") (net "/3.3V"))
 (segment (start 32 44.7) (end 33.7 44.7) (width 1) (layer "F.Cu") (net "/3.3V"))
 (segment (start 39.6375 45.696) (end 39.6375 42.8375) (width 0.5) (layer "F.Cu") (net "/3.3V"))
 (segment (start 37.6 31.2) (end 32 36.8) (width 1) (layer "F.Cu") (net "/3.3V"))
 (segment (start 64.8 47.082) (end 67.282 47.082) (width 1) (layer "F.Cu") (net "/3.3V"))
 (segment (start 58.5 51) (end 60.3625 49.1375) (width 0.5) (layer "F.Cu") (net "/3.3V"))
 (segment (start 62.0375 47.082) (end 61.636 47.082) (width 0.25) (layer "F.Cu") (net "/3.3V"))
 (segment (start 33.7 44.7) (end 35.6 42.8) (width 1) (layer "F.Cu") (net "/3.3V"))
 (segment (start 69 49.5) (end 69 48.8) (width 1) (layer "F.Cu") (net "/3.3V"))
 (segment (start 66.2 47.082) (end 66 46.882) (width 1) (layer "F.Cu") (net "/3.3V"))
 (segment (start 66 46.882) (end 66 35) (width 1) (layer "F.Cu") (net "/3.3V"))
 (segment (start 58 51) (end 49.6 51) (width 1) (layer "F.Cu") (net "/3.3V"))
 (segment (start 63.795398 47.082) (end 63.795221 47.081823) (width 0.25) (layer "F.Cu") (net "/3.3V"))
 (segment (start 62.2 31.2) (end 37.6 31.2) (width 1) (layer "F.Cu") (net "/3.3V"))
 (segment (start 52.7 36.61) (end 51.54 35.45) (width 1) (layer "F.Cu") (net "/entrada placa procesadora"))
 (segment (start 52.7 45.8) (end 52.7 36.61) (width 1) (layer "F.Cu") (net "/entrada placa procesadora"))
 (segment (start 40.718 46.518) (end 39.6375 46.518) (width 0.5) (layer "F.Cu") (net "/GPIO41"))
 (segment (start 41.8 49.2) (end 41.8 47.6) (width 0.5) (layer "F.Cu") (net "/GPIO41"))
 (segment (start 56.364 49) (end 58.282 47.082) (width 1) (layer "F.Cu") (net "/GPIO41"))
 (segment (start 43.4 50.8) (end 43.4 56.85) (width 1) (layer "F.Cu") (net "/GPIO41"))
 (segment (start 45.2 49) (end 56.364 49) (width 1) (layer "F.Cu") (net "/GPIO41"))
 (segment (start 43.4 50.8) (end 45.2 49) (width 1) (layer "F.Cu") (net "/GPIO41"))
 (segment (start 41.8 49.2) (end 43.4 50.8) (width 1) (layer "F.Cu") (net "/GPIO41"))
 (segment (start 43.4 56.85) (end 45.2 58.65) (width 1) (layer "F.Cu") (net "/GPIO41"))
 (segment (start 60.3625 47.082) (end 58.282 47.082) (width 0.5) (layer "F.Cu") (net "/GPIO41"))
 (segment (start 41.8 47.6) (end 40.718 46.518) (width 0.5) (layer "F.Cu") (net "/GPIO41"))
 (segment (start 36.4 62.8) (end 28.6 55) (width 1) (layer "F.Cu") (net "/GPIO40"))
 (segment (start 48.8 62.8) (end 36.4 62.8) (width 1) (layer "F.Cu") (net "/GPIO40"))
 (segment (start 28.6 55) (end 28.6 49.2) (width 1) (layer "F.Cu") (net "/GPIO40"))
 (segment (start 37.9625 45.696) (end 36.104 45.696) (width 0.5) (layer "F.Cu") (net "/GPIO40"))
 (segment (start 30.8 47) (end 34.8 47) (width 1) (layer "F.Cu") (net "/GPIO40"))
 (segment (start 50.4 55.8) (end 50.4 58.53) (width 1) (layer "F.Cu") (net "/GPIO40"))
 (segment (start 50.28 58.65) (end 50.2 58.73) (width 1) (layer "F.Cu") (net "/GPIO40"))
 (segment (start 62.0375 47.904) (end 62.0375 51.1625) (width 0.5) (layer "F.Cu") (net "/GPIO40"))
 (segment (start 50.2 61.4) (end 48.8 62.8) (width 1) (layer "F.Cu") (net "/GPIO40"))
 (segment (start 53 53.2) (end 50.4 55.8) (width 1) (layer "F.Cu") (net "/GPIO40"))
 (segment (start 60 53.2) (end 53 53.2) (width 1) (layer "F.Cu") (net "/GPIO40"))
 (segment (start 50.2 58.73) (end 50.2 61.4) (width 1) (layer "F.Cu") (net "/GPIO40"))
 (segment (start 62 51.2) (end 60 53.2) (width 1) (layer "F.Cu") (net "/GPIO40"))
 (segment (start 36.104 45.696) (end 34.8 47) (width 0.5) (layer "F.Cu") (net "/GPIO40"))
 (segment (start 28.6 49.2) (end 30.8 47) (width 1) (layer "F.Cu") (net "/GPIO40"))
 (segment (start 62.0375 51.1625) (end 62 51.2) (width 0.5) (layer "F.Cu") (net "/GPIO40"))
 (segment (start 50.4 58.53) (end 50.28 58.65) (width 1) (layer "F.Cu") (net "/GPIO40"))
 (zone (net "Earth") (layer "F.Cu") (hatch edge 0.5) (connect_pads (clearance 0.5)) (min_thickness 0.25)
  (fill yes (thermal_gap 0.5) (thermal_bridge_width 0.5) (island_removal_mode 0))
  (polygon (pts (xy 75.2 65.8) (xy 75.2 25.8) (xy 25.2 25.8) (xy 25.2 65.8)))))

